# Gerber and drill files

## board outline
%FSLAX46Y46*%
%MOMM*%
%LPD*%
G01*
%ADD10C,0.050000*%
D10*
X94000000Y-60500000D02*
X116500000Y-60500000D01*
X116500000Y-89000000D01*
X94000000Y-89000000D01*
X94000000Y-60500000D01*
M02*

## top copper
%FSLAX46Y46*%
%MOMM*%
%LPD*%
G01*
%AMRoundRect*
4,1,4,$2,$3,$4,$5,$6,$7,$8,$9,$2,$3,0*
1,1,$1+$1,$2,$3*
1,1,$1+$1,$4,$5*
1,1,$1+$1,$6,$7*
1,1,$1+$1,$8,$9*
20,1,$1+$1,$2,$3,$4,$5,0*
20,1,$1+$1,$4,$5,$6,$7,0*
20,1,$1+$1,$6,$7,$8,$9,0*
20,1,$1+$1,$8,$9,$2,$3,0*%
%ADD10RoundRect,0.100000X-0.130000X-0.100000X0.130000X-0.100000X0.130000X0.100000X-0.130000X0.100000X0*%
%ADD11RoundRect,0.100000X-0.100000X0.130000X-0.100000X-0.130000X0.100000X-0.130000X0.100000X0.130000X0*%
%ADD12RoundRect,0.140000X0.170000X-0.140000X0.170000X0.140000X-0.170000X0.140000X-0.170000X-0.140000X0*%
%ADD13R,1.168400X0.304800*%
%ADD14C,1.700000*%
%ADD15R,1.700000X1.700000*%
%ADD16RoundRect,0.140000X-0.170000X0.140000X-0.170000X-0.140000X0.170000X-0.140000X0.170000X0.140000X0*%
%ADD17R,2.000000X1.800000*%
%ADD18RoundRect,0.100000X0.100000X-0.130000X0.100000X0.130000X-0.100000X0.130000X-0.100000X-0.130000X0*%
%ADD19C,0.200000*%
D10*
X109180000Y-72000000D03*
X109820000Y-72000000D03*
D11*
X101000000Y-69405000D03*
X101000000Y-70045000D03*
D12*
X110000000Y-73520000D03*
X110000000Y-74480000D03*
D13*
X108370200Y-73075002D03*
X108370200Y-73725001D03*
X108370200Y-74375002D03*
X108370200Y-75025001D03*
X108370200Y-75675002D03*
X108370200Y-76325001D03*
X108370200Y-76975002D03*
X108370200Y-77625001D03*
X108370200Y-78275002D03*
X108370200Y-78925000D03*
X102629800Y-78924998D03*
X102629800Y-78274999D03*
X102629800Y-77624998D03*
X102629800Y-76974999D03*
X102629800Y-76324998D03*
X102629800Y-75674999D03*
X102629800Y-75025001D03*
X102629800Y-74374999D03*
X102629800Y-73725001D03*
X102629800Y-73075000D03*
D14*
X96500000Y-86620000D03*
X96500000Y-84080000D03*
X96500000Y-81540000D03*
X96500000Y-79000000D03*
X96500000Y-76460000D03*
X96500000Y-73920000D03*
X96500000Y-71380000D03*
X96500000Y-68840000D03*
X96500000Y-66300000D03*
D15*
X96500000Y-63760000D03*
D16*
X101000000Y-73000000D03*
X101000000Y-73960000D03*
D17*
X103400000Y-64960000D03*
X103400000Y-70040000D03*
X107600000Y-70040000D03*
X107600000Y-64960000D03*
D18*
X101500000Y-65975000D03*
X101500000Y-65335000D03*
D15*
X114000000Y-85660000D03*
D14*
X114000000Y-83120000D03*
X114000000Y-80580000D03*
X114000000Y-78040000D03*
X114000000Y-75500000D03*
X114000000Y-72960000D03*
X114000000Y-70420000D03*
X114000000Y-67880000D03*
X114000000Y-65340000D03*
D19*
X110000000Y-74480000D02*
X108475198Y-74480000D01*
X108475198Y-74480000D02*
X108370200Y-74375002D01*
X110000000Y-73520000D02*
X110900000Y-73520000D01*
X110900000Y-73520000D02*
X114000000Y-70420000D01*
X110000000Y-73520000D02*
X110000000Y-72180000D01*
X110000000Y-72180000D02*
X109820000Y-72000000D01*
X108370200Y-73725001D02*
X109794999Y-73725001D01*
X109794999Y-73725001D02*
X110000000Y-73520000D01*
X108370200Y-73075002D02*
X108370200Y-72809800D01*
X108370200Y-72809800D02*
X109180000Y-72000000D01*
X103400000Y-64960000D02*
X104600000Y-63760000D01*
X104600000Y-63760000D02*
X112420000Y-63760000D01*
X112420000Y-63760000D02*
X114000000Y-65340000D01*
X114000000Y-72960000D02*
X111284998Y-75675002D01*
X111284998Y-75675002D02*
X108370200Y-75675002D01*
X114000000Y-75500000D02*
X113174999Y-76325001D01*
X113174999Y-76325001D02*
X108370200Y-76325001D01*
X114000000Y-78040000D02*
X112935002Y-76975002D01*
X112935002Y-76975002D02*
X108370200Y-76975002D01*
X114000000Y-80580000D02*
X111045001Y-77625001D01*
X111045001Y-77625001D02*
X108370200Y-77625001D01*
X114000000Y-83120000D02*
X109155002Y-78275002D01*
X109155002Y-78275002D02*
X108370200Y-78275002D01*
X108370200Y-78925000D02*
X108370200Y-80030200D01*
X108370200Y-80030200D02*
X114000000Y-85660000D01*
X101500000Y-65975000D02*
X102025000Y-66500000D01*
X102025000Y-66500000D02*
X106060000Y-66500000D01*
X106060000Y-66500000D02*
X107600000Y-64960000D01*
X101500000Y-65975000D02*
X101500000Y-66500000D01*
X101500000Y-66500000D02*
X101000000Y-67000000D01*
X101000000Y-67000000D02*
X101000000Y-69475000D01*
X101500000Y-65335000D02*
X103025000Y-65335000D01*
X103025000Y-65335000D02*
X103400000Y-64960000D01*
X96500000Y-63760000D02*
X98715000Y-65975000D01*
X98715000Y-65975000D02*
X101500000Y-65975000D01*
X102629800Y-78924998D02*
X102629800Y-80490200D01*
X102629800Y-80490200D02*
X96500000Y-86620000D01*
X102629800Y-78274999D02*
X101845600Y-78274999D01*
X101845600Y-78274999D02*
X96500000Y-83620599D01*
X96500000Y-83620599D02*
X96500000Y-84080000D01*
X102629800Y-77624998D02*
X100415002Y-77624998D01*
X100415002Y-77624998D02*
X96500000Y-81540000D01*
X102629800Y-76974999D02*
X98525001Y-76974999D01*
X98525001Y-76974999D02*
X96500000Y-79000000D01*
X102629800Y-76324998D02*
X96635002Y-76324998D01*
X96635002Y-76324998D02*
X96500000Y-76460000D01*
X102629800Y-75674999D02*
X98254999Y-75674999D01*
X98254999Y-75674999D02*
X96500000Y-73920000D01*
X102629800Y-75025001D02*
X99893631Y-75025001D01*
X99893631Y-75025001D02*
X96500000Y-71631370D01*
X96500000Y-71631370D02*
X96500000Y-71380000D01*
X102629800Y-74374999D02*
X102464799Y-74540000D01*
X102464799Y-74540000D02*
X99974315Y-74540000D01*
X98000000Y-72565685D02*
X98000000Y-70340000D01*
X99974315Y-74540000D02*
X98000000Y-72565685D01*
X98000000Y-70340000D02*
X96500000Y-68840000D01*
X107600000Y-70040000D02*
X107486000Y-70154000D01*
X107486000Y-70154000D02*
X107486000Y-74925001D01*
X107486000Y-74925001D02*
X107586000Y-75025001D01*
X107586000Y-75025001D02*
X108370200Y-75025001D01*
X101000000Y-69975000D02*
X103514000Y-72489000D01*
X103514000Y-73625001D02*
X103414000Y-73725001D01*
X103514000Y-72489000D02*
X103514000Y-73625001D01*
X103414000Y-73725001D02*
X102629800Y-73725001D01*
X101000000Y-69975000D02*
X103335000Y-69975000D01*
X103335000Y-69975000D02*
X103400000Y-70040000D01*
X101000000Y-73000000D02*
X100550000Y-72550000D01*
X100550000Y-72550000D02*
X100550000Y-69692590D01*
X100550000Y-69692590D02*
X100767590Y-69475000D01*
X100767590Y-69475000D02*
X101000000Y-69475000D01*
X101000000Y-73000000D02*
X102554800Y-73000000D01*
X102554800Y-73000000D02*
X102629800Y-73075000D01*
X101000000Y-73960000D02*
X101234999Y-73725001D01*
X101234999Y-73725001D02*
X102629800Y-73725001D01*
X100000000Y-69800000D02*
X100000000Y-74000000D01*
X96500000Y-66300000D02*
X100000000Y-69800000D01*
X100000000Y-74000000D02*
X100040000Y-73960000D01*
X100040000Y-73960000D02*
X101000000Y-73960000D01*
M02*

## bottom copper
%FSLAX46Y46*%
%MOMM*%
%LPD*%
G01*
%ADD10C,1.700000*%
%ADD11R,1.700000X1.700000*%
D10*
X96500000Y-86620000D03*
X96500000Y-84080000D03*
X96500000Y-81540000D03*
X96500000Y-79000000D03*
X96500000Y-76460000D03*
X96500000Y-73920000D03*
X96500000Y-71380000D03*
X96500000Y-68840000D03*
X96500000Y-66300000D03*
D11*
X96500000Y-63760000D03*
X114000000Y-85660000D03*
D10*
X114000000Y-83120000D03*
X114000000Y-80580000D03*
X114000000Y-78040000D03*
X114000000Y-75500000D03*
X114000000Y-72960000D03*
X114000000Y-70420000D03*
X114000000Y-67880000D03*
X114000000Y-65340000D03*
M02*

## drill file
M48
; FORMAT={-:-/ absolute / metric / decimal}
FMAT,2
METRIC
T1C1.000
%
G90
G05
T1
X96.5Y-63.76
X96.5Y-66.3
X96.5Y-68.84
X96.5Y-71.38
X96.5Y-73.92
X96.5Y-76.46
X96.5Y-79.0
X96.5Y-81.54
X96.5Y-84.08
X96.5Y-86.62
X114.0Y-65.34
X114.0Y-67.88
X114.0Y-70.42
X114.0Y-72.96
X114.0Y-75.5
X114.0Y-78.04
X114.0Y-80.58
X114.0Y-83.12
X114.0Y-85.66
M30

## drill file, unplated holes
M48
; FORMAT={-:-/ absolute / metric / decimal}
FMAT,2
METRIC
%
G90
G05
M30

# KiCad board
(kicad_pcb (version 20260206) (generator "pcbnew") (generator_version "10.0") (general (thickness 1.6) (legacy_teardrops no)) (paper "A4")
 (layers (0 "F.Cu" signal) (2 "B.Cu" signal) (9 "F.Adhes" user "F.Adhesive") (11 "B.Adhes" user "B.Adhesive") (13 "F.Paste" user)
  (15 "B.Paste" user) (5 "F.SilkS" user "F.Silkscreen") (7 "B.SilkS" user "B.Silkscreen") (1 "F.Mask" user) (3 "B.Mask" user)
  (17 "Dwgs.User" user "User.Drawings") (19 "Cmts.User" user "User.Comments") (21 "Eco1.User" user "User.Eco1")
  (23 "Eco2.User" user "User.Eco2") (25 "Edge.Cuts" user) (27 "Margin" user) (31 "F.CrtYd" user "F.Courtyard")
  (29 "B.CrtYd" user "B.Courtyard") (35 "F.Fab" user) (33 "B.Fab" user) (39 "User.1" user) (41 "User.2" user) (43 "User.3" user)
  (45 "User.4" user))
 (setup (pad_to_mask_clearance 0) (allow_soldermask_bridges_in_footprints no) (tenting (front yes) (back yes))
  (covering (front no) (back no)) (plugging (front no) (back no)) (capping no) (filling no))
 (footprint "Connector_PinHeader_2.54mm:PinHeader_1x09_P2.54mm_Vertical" (layer "F.Cu") (at 114 85.66 180)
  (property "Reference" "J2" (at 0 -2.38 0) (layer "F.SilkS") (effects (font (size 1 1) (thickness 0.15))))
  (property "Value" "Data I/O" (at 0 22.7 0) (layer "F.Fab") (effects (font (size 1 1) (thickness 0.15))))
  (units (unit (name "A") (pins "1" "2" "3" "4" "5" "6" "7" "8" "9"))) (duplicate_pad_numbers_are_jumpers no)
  (pad "1" thru_hole rect (at 0 0 180) (size 1.7 1.7) (drill 1) (layers "*.Cu" "*.Mask") (remove_unused_layers no) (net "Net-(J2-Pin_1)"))
  (pad "2" thru_hole circle (at 0 2.54 180) (size 1.7 1.7) (drill 1) (layers "*.Cu" "*.Mask") (remove_unused_layers no)
   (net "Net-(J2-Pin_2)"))
  (pad "3" thru_hole circle (at 0 5.08 180) (size 1.7 1.7) (drill 1) (layers "*.Cu" "*.Mask") (remove_unused_layers no)
   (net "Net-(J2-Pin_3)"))
  (pad "4" thru_hole circle (at 0 7.62 180) (size 1.7 1.7) (drill 1) (layers "*.Cu" "*.Mask") (remove_unused_layers no)
   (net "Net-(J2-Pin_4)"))
  (pad "5" thru_hole circle (at 0 10.16 180) (size 1.7 1.7) (drill 1) (layers "*.Cu" "*.Mask") (remove_unused_layers no)
   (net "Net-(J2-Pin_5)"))
  (pad "6" thru_hole circle (at 0 12.7 180) (size 1.7 1.7) (drill 1) (layers "*.Cu" "*.Mask") (remove_unused_layers no)
   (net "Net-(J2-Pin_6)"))
  (pad "7" thru_hole circle (at 0 15.24 180) (size 1.7 1.7) (drill 1) (layers "*.Cu" "*.Mask") (remove_unused_layers no)
   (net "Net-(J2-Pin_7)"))
  (pad "8" thru_hole circle (at 0 17.78 180) (size 1.7 1.7) (drill 1) (layers "*.Cu" "*.Mask") (remove_unused_layers no)
   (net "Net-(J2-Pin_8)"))
  (pad "9" thru_hole circle (at 0 20.32 180) (size 1.7 1.7) (drill 1) (layers "*.Cu" "*.Mask") (remove_unused_layers no)
   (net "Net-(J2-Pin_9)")))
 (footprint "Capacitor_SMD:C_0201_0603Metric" (layer "F.Cu") (at 109.5 72)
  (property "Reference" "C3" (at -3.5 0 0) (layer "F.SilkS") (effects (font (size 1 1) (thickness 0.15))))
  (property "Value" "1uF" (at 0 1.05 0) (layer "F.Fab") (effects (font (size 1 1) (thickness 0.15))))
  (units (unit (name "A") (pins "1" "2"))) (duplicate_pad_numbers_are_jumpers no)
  (pad "" smd roundrect (at -0.345 0) (size 0.318 0.36) (layers "F.Paste") (roundrect_rratio 0.25))
  (pad "" smd roundrect (at 0.345 0) (size 0.318 0.36) (layers "F.Paste") (roundrect_rratio 0.25))
  (pad "1" smd roundrect (at -0.32 0) (size 0.46 0.4) (layers "F.Cu" "F.Mask") (roundrect_rratio 0.25) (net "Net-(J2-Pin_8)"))
  (pad "2" smd roundrect (at 0.32 0) (size 0.46 0.4) (layers "F.Cu" "F.Mask") (roundrect_rratio 0.25) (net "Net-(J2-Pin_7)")))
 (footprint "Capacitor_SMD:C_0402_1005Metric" (layer "F.Cu") (at 101 73.48 -90)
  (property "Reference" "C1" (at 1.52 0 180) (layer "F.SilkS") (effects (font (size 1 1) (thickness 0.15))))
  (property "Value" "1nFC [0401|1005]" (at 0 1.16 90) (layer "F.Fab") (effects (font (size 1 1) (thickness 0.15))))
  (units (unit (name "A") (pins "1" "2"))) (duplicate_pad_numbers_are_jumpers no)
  (pad "1" smd roundrect (at -0.48 0 270) (size 0.56 0.62) (layers "F.Cu" "F.Mask" "F.Paste") (roundrect_rratio 0.25) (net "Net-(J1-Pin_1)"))
  (pad "2" smd roundrect (at 0.48 0 270) (size 0.56 0.62) (layers "F.Cu" "F.Mask" "F.Paste") (roundrect_rratio 0.25) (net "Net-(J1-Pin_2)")))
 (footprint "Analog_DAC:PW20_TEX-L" (layer "F.Cu") (at 105.5 76)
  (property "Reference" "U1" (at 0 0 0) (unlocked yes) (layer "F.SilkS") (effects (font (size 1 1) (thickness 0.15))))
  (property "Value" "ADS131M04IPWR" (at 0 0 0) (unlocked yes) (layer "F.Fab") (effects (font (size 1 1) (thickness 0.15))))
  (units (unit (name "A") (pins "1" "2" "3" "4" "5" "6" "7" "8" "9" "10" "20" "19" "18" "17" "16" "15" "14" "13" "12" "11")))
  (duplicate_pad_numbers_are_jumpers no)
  (pad "1" smd rect (at -2.8702 -2.925) (size 1.1684 0.3048) (layers "F.Cu" "F.Mask" "F.Paste") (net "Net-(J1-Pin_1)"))
  (pad "2" smd rect (at -2.8702 -2.274999) (size 1.1684 0.3048) (layers "F.Cu" "F.Mask" "F.Paste") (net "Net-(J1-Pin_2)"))
  (pad "3" smd rect (at -2.8702 -1.625001) (size 1.1684 0.3048) (layers "F.Cu" "F.Mask" "F.Paste") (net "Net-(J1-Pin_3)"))
  (pad "4" smd rect (at -2.8702 -0.974999) (size 1.1684 0.3048) (layers "F.Cu" "F.Mask" "F.Paste") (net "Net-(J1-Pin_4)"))
  (pad "5" smd rect (at -2.8702 -0.325001) (size 1.1684 0.3048) (layers "F.Cu" "F.Mask" "F.Paste") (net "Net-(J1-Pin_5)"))
  (pad "6" smd rect (at -2.8702 0.324998) (size 1.1684 0.3048) (layers "F.Cu" "F.Mask" "F.Paste") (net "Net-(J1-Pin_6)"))
  (pad "7" smd rect (at -2.8702 0.974999) (size 1.1684 0.3048) (layers "F.Cu" "F.Mask" "F.Paste") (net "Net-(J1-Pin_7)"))
  (pad "8" smd rect (at -2.8702 1.624998) (size 1.1684 0.3048) (layers "F.Cu" "F.Mask" "F.Paste") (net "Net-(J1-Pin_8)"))
  (pad "9" smd rect (at -2.8702 2.274999) (size 1.1684 0.3048) (layers "F.Cu" "F.Mask" "F.Paste") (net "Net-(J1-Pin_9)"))
  (pad "10" smd rect (at -2.8702 2.924998) (size 1.1684 0.3048) (layers "F.Cu" "F.Mask" "F.Paste") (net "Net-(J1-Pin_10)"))
  (pad "11" smd rect (at 2.8702 2.925) (size 1.1684 0.3048) (layers "F.Cu" "F.Mask" "F.Paste") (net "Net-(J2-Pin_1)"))
  (pad "12" smd rect (at 2.8702 2.275002) (size 1.1684 0.3048) (layers "F.Cu" "F.Mask" "F.Paste") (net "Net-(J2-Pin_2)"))
  (pad "13" smd rect (at 2.8702 1.625001) (size 1.1684 0.3048) (layers "F.Cu" "F.Mask" "F.Paste") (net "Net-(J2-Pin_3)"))
  (pad "14" smd rect (at 2.8702 0.975002) (size 1.1684 0.3048) (layers "F.Cu" "F.Mask" "F.Paste") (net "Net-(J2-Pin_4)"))
  (pad "15" smd rect (at 2.8702 0.325001) (size 1.1684 0.3048) (layers "F.Cu" "F.Mask" "F.Paste") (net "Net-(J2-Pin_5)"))
  (pad "16" smd rect (at 2.8702 -0.324998) (size 1.1684 0.3048) (layers "F.Cu" "F.Mask" "F.Paste") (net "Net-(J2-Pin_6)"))
  (pad "17" smd rect (at 2.8702 -0.974999) (size 1.1684 0.3048) (layers "F.Cu" "F.Mask" "F.Paste") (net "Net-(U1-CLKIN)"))
  (pad "18" smd rect (at 2.8702 -1.624998) (size 1.1684 0.3048) (layers "F.Cu" "F.Mask" "F.Paste") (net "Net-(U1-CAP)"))
  (pad "19" smd rect (at 2.8702 -2.274999) (size 1.1684 0.3048) (layers "F.Cu" "F.Mask" "F.Paste") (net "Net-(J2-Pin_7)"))
  (pad "20" smd rect (at 2.8702 -2.924998) (size 1.1684 0.3048) (layers "F.Cu" "F.Mask" "F.Paste") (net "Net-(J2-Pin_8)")))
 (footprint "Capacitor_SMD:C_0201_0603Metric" (layer "F.Cu") (at 101 69.725 -90)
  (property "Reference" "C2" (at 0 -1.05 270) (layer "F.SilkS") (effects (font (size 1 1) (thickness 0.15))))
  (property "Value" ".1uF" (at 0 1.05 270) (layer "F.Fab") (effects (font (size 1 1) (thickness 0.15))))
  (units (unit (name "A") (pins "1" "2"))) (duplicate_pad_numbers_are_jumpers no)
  (pad "" smd roundrect (at -0.345 0 270) (size 0.318 0.36) (layers "F.Paste") (roundrect_rratio 0.25))
  (pad "" smd roundrect (at 0.345 0 270) (size 0.318 0.36) (layers "F.Paste") (roundrect_rratio 0.25))
  (pad "1" smd roundrect (at -0.32 0 270) (size 0.46 0.4) (layers "F.Cu" "F.Mask") (roundrect_rratio 0.25) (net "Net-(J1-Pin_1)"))
  (pad "2" smd roundrect (at 0.32 0 270) (size 0.46 0.4) (layers "F.Cu" "F.Mask") (roundrect_rratio 0.25) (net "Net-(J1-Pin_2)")))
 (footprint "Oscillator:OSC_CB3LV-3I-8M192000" (layer "F.Cu") (at 105.5 67.5)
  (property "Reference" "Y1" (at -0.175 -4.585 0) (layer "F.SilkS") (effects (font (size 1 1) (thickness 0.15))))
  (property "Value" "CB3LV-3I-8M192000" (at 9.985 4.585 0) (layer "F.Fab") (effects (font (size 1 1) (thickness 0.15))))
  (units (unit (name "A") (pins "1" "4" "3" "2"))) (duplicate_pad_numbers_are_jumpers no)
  (pad "1" smd rect (at -2.1 -2.54) (size 2 1.8) (layers "F.Cu" "F.Mask" "F.Paste") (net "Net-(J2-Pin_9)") (solder_mask_margin 0.102))
  (pad "2" smd rect (at -2.1 2.54) (size 2 1.8) (layers "F.Cu" "F.Mask" "F.Paste") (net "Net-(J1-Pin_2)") (solder_mask_margin 0.102))
  (pad "3" smd rect (at 2.1 2.54) (size 2 1.8) (layers "F.Cu" "F.Mask" "F.Paste") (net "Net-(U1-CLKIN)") (solder_mask_margin 0.102))
  (pad "4" smd rect (at 2.1 -2.54) (size 2 1.8) (layers "F.Cu" "F.Mask" "F.Paste") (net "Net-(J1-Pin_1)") (solder_mask_margin 0.102)))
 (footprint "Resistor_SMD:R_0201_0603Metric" (layer "F.Cu") (at 101.5 65.655 90)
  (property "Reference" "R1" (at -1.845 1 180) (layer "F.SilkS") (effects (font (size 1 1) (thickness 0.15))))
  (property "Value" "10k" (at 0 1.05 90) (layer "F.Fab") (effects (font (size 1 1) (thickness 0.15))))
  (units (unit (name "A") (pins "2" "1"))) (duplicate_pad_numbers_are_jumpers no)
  (pad "" smd roundrect (at -0.345 0 90) (size 0.318 0.36) (layers "F.Paste") (roundrect_rratio 0.25))
  (pad "" smd roundrect (at 0.345 0 90) (size 0.318 0.36) (layers "F.Paste") (roundrect_rratio 0.25))
  (pad "1" smd roundrect (at -0.32 0 90) (size 0.46 0.4) (layers "F.Cu" "F.Mask") (roundrect_rratio 0.25) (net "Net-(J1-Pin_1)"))
  (pad "2" smd roundrect (at 0.32 0 90) (size 0.46 0.4) (layers "F.Cu" "F.Mask") (roundrect_rratio 0.25) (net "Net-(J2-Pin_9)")))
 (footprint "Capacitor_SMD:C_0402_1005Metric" (layer "F.Cu") (at 110 74 90)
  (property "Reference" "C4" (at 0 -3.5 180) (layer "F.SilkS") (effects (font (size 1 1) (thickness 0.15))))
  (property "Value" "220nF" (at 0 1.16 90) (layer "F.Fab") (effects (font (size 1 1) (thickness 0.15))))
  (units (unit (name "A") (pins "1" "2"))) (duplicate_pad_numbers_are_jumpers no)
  (pad "1" smd roundrect (at -0.48 0 90) (size 0.56 0.62) (layers "F.Cu" "F.Mask" "F.Paste") (roundrect_rratio 0.25) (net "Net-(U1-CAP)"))
  (pad "2" smd roundrect (at 0.48 0 90) (size 0.56 0.62) (layers "F.Cu" "F.Mask" "F.Paste") (roundrect_rratio 0.25) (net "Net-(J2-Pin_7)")))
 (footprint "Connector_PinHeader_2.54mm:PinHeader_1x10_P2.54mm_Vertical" (layer "F.Cu") (at 96.5 63.76)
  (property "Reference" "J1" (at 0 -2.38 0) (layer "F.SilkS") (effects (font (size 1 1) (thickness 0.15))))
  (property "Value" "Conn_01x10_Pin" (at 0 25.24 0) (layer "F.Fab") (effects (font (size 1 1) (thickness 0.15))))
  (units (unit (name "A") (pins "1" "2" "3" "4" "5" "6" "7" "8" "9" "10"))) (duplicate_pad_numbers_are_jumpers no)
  (pad "1" thru_hole rect (at 0 0) (size 1.7 1.7) (drill 1) (layers "*.Cu" "*.Mask") (remove_unused_layers no) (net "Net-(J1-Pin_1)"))
  (pad "2" thru_hole circle (at 0 2.54) (size 1.7 1.7) (drill 1) (layers "*.Cu" "*.Mask") (remove_unused_layers no) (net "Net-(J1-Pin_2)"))
  (pad "3" thru_hole circle (at 0 5.08) (size 1.7 1.7) (drill 1) (layers "*.Cu" "*.Mask") (remove_unused_layers no) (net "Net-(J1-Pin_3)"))
  (pad "4" thru_hole circle (at 0 7.62) (size 1.7 1.7) (drill 1) (layers "*.Cu" "*.Mask") (remove_unused_layers no) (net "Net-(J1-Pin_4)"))
  (pad "5" thru_hole circle (at 0 10.16) (size 1.7 1.7) (drill 1) (layers "*.Cu" "*.Mask") (remove_unused_layers no) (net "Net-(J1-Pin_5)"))
  (pad "6" thru_hole circle (at 0 12.7) (size 1.7 1.7) (drill 1) (layers "*.Cu" "*.Mask") (remove_unused_layers no) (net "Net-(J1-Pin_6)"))
  (pad "7" thru_hole circle (at 0 15.24) (size 1.7 1.7) (drill 1) (layers "*.Cu" "*.Mask") (remove_unused_layers no) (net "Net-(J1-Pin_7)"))
  (pad "8" thru_hole circle (at 0 17.78) (size 1.7 1.7) (drill 1) (layers "*.Cu" "*.Mask") (remove_unused_layers no) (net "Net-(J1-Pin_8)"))
  (pad "9" thru_hole circle (at 0 20.32) (size 1.7 1.7) (drill 1) (layers "*.Cu" "*.Mask") (remove_unused_layers no) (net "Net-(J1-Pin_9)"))
  (pad "10" thru_hole circle (at 0 22.86) (size 1.7 1.7) (drill 1) (layers "*.Cu" "*.Mask") (remove_unused_layers no)
   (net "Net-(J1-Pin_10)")))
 (gr_rect (start 94 60.5) (end 116.5 89) (stroke (width 0.05) (type default)) (fill no) (layer "Edge.Cuts"))
 (segment (start 108.3702 80.0302) (end 114 85.66) (width 0.2) (layer "F.Cu") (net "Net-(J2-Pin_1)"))
 (segment (start 108.3702 78.925) (end 108.3702 80.0302) (width 0.2) (layer "F.Cu") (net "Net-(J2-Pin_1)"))
 (segment (start 114 83.12) (end 109.155002 78.275002) (width 0.2) (layer "F.Cu") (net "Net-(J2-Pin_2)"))
 (segment (start 109.155002 78.275002) (end 108.3702 78.275002) (width 0.2) (layer "F.Cu") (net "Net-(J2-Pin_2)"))
 (segment (start 111.045001 77.625001) (end 108.3702 77.625001) (width 0.2) (layer "F.Cu") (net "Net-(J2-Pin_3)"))
 (segment (start 114 80.58) (end 111.045001 77.625001) (width 0.2) (layer "F.Cu") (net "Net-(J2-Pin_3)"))
 (segment (start 114 78.04) (end 112.935002 76.975002) (width 0.2) (layer "F.Cu") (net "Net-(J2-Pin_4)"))
 (segment (start 112.935002 76.975002) (end 108.3702 76.975002) (width 0.2) (layer "F.Cu") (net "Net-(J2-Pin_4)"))
 (segment (start 114 75.5) (end 113.174999 76.325001) (width 0.2) (layer "F.Cu") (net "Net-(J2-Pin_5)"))
 (segment (start 113.174999 76.325001) (end 108.3702 76.325001) (width 0.2) (layer "F.Cu") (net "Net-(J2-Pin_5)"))
 (segment (start 111.284998 75.675002) (end 108.3702 75.675002) (width 0.2) (layer "F.Cu") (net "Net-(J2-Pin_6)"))
 (segment (start 114 72.96) (end 111.284998 75.675002) (width 0.2) (layer "F.Cu") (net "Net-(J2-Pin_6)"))
 (segment (start 110 73.52) (end 110 72.18) (width 0.2) (layer "F.Cu") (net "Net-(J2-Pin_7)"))
 (segment (start 110 73.52) (end 110.9 73.52) (width 0.2) (layer "F.Cu") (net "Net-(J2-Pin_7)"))
 (segment (start 110 72.18) (end 109.82 72) (width 0.2) (layer "F.Cu") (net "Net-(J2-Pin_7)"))
 (segment (start 108.3702 73.725001) (end 109.794999 73.725001) (width 0.2) (layer "F.Cu") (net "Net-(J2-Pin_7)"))
 (segment (start 109.794999 73.725001) (end 110 73.52) (width 0.2) (layer "F.Cu") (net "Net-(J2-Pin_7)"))
 (segment (start 110.9 73.52) (end 114 70.42) (width 0.2) (layer "F.Cu") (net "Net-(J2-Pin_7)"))
 (segment (start 108.3702 73.075002) (end 108.3702 72.8098) (width 0.2) (layer "F.Cu") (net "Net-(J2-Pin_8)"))
 (segment (start 108.3702 72.8098) (end 109.18 72) (width 0.2) (layer "F.Cu") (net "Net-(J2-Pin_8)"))
 (segment (start 112.42 63.76) (end 114 65.34) (width 0.2) (layer "F.Cu") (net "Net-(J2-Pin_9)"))
 (segment (start 101.5 65.335) (end 103.025 65.335) (width 0.2) (layer "F.Cu") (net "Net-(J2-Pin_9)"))
 (segment (start 103.4 64.96) (end 104.6 63.76) (width 0.2) (layer "F.Cu") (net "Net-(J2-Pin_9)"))
 (segment (start 104.6 63.76) (end 112.42 63.76) (width 0.2) (layer "F.Cu") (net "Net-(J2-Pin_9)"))
 (segment (start 103.025 65.335) (end 103.4 64.96) (width 0.2) (layer "F.Cu") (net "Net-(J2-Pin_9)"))
 (segment (start 96.5 63.76) (end 98.715 65.975) (width 0.2) (layer "F.Cu") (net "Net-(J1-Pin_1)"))
 (segment (start 101.5 66.5) (end 101 67) (width 0.2) (layer "F.Cu") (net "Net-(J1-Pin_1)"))
 (segment (start 101 73) (end 100.55 72.55) (width 0.2) (layer "F.Cu") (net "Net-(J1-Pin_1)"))
 (segment (start 102.025 66.5) (end 106.06 66.5) (width 0.2) (layer "F.Cu") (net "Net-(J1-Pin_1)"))
 (segment (start 101.5 65.975) (end 102.025 66.5) (width 0.2) (layer "F.Cu") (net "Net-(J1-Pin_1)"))
 (segment (start 98.715 65.975) (end 101.5 65.975) (width 0.2) (layer "F.Cu") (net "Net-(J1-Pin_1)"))
 (segment (start 101.5 65.975) (end 101.5 66.5) (width 0.2) (layer "F.Cu") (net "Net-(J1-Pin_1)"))
 (segment (start 100.55 69.69259) (end 100.76759 69.475) (width 0.2) (layer "F.Cu") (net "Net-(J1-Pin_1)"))
 (segment (start 100.55 72.55) (end 100.55 69.69259) (width 0.2) (layer "F.Cu") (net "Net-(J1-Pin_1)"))
 (segment (start 100.76759 69.475) (end 101 69.475) (width 0.2) (layer "F.Cu") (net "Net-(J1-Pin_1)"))
 (segment (start 102.5548 73) (end 102.6298 73.075) (width 0.2) (layer "F.Cu") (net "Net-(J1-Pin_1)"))
 (segment (start 101 73) (end 102.5548 73) (width 0.2) (layer "F.Cu") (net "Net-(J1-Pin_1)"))
 (segment (start 101 67) (end 101 69.475) (width 0.2) (layer "F.Cu") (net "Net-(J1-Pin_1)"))
 (segment (start 106.06 66.5) (end 107.6 64.96) (width 0.2) (layer "F.Cu") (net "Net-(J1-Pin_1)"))
 (segment (start 101.234999 73.725001) (end 102.6298 73.725001) (width 0.2) (layer "F.Cu") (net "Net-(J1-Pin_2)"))
 (segment (start 96.5 66.3) (end 100 69.8) (width 0.2) (layer "F.Cu") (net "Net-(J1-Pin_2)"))
 (segment (start 103.335 69.975) (end 103.4 70.04) (width 0.2) (layer "F.Cu") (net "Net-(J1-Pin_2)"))
 (segment (start 101 73.96) (end 101.234999 73.725001) (width 0.2) (layer "F.Cu") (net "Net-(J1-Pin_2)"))
 (segment (start 100.04 73.96) (end 101 73.96) (width 0.2) (layer "F.Cu") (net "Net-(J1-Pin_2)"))
 (segment (start 103.514 72.489) (end 103.514 73.625001) (width 0.2) (layer "F.Cu") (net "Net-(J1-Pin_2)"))
 (segment (start 100 74) (end 100.04 73.96) (width 0.2) (layer "F.Cu") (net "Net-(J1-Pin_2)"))
 (segment (start 101 69.975) (end 103.335 69.975) (width 0.2) (layer "F.Cu") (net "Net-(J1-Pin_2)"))
 (segment (start 103.414 73.725001) (end 102.6298 73.725001) (width 0.2) (layer "F.Cu") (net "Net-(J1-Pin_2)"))
 (segment (start 101 69.975) (end 103.514 72.489) (width 0.2) (layer "F.Cu") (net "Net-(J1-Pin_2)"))
 (segment (start 103.514 73.625001) (end 103.414 73.725001) (width 0.2) (layer "F.Cu") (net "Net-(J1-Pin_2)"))
 (segment (start 100 69.8) (end 100 74) (width 0.2) (layer "F.Cu") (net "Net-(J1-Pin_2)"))
 (segment (start 99.974315 74.54) (end 98 72.565685) (width 0.2) (layer "F.Cu") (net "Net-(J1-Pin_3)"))
 (segment (start 102.464799 74.54) (end 99.974315 74.54) (width 0.2) (layer "F.Cu") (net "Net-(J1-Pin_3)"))
 (segment (start 98 72.565685) (end 98 70.34) (width 0.2) (layer "F.Cu") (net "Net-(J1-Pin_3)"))
 (segment (start 98 70.34) (end 96.5 68.84) (width 0.2) (layer "F.Cu") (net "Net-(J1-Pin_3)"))
 (segment (start 102.6298 74.374999) (end 102.464799 74.54) (width 0.2) (layer "F.Cu") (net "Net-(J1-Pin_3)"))
 (segment (start 102.6298 75.025001) (end 99.893631 75.025001) (width 0.2) (layer "F.Cu") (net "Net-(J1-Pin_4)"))
 (segment (start 96.5 71.63137) (end 96.5 71.38) (width 0.2) (layer "F.Cu") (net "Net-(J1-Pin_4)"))
 (segment (start 99.893631 75.025001) (end 96.5 71.63137) (width 0.2) (layer "F.Cu") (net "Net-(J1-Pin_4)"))
 (segment (start 98.254999 75.674999) (end 96.5 73.92) (width 0.2) (layer "F.Cu") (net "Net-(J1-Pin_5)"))
 (segment (start 102.6298 75.674999) (end 98.254999 75.674999) (width 0.2) (layer "F.Cu") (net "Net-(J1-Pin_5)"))
 (segment (start 96.635002 76.324998) (end 96.5 76.46) (width 0.2) (layer "F.Cu") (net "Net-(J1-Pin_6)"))
 (segment (start 102.6298 76.324998) (end 96.635002 76.324998) (width 0.2) (layer "F.Cu") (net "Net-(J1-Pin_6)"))
 (segment (start 102.6298 76.974999) (end 98.525001 76.974999) (width 0.2) (layer "F.Cu") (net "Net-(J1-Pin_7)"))
 (segment (start 98.525001 76.974999) (end 96.5 79) (width 0.2) (layer "F.Cu") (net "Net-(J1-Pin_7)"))
 (segment (start 100.415002 77.624998) (end 96.5 81.54) (width 0.2) (layer "F.Cu") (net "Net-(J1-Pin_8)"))
 (segment (start 102.6298 77.624998) (end 100.415002 77.624998) (width 0.2) (layer "F.Cu") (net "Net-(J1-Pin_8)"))
 (segment (start 102.6298 78.274999) (end 101.8456 78.274999) (width 0.2) (layer "F.Cu") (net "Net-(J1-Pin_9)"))
 (segment (start 101.8456 78.274999) (end 96.5 83.620599) (width 0.2) (layer "F.Cu") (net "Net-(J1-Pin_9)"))
 (segment (start 96.5 83.620599) (end 96.5 84.08) (width 0.2) (layer "F.Cu") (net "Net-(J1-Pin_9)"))
 (segment (start 102.6298 80.4902) (end 96.5 86.62) (width 0.2) (layer "F.Cu") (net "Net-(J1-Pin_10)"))
 (segment (start 102.6298 78.924998) (end 102.6298 80.4902) (width 0.2) (layer "F.Cu") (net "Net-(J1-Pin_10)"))
 (segment (start 107.486 74.925001) (end 107.586 75.025001) (width 0.2) (layer "F.Cu") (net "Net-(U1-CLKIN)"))
 (segment (start 107.586 75.025001) (end 108.3702 75.025001) (width 0.2) (layer "F.Cu") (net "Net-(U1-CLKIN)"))
 (segment (start 107.486 70.154) (end 107.486 74.925001) (width 0.2) (layer "F.Cu") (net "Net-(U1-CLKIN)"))
 (segment (start 107.6 70.04) (end 107.486 70.154) (width 0.2) (layer "F.Cu") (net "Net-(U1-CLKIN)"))
 (segment (start 110 74.48) (end 108.475198 74.48) (width 0.2) (layer "F.Cu") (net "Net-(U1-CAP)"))
 (segment (start 108.475198 74.48) (end 108.3702 74.375002) (width 0.2) (layer "F.Cu") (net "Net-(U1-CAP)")))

